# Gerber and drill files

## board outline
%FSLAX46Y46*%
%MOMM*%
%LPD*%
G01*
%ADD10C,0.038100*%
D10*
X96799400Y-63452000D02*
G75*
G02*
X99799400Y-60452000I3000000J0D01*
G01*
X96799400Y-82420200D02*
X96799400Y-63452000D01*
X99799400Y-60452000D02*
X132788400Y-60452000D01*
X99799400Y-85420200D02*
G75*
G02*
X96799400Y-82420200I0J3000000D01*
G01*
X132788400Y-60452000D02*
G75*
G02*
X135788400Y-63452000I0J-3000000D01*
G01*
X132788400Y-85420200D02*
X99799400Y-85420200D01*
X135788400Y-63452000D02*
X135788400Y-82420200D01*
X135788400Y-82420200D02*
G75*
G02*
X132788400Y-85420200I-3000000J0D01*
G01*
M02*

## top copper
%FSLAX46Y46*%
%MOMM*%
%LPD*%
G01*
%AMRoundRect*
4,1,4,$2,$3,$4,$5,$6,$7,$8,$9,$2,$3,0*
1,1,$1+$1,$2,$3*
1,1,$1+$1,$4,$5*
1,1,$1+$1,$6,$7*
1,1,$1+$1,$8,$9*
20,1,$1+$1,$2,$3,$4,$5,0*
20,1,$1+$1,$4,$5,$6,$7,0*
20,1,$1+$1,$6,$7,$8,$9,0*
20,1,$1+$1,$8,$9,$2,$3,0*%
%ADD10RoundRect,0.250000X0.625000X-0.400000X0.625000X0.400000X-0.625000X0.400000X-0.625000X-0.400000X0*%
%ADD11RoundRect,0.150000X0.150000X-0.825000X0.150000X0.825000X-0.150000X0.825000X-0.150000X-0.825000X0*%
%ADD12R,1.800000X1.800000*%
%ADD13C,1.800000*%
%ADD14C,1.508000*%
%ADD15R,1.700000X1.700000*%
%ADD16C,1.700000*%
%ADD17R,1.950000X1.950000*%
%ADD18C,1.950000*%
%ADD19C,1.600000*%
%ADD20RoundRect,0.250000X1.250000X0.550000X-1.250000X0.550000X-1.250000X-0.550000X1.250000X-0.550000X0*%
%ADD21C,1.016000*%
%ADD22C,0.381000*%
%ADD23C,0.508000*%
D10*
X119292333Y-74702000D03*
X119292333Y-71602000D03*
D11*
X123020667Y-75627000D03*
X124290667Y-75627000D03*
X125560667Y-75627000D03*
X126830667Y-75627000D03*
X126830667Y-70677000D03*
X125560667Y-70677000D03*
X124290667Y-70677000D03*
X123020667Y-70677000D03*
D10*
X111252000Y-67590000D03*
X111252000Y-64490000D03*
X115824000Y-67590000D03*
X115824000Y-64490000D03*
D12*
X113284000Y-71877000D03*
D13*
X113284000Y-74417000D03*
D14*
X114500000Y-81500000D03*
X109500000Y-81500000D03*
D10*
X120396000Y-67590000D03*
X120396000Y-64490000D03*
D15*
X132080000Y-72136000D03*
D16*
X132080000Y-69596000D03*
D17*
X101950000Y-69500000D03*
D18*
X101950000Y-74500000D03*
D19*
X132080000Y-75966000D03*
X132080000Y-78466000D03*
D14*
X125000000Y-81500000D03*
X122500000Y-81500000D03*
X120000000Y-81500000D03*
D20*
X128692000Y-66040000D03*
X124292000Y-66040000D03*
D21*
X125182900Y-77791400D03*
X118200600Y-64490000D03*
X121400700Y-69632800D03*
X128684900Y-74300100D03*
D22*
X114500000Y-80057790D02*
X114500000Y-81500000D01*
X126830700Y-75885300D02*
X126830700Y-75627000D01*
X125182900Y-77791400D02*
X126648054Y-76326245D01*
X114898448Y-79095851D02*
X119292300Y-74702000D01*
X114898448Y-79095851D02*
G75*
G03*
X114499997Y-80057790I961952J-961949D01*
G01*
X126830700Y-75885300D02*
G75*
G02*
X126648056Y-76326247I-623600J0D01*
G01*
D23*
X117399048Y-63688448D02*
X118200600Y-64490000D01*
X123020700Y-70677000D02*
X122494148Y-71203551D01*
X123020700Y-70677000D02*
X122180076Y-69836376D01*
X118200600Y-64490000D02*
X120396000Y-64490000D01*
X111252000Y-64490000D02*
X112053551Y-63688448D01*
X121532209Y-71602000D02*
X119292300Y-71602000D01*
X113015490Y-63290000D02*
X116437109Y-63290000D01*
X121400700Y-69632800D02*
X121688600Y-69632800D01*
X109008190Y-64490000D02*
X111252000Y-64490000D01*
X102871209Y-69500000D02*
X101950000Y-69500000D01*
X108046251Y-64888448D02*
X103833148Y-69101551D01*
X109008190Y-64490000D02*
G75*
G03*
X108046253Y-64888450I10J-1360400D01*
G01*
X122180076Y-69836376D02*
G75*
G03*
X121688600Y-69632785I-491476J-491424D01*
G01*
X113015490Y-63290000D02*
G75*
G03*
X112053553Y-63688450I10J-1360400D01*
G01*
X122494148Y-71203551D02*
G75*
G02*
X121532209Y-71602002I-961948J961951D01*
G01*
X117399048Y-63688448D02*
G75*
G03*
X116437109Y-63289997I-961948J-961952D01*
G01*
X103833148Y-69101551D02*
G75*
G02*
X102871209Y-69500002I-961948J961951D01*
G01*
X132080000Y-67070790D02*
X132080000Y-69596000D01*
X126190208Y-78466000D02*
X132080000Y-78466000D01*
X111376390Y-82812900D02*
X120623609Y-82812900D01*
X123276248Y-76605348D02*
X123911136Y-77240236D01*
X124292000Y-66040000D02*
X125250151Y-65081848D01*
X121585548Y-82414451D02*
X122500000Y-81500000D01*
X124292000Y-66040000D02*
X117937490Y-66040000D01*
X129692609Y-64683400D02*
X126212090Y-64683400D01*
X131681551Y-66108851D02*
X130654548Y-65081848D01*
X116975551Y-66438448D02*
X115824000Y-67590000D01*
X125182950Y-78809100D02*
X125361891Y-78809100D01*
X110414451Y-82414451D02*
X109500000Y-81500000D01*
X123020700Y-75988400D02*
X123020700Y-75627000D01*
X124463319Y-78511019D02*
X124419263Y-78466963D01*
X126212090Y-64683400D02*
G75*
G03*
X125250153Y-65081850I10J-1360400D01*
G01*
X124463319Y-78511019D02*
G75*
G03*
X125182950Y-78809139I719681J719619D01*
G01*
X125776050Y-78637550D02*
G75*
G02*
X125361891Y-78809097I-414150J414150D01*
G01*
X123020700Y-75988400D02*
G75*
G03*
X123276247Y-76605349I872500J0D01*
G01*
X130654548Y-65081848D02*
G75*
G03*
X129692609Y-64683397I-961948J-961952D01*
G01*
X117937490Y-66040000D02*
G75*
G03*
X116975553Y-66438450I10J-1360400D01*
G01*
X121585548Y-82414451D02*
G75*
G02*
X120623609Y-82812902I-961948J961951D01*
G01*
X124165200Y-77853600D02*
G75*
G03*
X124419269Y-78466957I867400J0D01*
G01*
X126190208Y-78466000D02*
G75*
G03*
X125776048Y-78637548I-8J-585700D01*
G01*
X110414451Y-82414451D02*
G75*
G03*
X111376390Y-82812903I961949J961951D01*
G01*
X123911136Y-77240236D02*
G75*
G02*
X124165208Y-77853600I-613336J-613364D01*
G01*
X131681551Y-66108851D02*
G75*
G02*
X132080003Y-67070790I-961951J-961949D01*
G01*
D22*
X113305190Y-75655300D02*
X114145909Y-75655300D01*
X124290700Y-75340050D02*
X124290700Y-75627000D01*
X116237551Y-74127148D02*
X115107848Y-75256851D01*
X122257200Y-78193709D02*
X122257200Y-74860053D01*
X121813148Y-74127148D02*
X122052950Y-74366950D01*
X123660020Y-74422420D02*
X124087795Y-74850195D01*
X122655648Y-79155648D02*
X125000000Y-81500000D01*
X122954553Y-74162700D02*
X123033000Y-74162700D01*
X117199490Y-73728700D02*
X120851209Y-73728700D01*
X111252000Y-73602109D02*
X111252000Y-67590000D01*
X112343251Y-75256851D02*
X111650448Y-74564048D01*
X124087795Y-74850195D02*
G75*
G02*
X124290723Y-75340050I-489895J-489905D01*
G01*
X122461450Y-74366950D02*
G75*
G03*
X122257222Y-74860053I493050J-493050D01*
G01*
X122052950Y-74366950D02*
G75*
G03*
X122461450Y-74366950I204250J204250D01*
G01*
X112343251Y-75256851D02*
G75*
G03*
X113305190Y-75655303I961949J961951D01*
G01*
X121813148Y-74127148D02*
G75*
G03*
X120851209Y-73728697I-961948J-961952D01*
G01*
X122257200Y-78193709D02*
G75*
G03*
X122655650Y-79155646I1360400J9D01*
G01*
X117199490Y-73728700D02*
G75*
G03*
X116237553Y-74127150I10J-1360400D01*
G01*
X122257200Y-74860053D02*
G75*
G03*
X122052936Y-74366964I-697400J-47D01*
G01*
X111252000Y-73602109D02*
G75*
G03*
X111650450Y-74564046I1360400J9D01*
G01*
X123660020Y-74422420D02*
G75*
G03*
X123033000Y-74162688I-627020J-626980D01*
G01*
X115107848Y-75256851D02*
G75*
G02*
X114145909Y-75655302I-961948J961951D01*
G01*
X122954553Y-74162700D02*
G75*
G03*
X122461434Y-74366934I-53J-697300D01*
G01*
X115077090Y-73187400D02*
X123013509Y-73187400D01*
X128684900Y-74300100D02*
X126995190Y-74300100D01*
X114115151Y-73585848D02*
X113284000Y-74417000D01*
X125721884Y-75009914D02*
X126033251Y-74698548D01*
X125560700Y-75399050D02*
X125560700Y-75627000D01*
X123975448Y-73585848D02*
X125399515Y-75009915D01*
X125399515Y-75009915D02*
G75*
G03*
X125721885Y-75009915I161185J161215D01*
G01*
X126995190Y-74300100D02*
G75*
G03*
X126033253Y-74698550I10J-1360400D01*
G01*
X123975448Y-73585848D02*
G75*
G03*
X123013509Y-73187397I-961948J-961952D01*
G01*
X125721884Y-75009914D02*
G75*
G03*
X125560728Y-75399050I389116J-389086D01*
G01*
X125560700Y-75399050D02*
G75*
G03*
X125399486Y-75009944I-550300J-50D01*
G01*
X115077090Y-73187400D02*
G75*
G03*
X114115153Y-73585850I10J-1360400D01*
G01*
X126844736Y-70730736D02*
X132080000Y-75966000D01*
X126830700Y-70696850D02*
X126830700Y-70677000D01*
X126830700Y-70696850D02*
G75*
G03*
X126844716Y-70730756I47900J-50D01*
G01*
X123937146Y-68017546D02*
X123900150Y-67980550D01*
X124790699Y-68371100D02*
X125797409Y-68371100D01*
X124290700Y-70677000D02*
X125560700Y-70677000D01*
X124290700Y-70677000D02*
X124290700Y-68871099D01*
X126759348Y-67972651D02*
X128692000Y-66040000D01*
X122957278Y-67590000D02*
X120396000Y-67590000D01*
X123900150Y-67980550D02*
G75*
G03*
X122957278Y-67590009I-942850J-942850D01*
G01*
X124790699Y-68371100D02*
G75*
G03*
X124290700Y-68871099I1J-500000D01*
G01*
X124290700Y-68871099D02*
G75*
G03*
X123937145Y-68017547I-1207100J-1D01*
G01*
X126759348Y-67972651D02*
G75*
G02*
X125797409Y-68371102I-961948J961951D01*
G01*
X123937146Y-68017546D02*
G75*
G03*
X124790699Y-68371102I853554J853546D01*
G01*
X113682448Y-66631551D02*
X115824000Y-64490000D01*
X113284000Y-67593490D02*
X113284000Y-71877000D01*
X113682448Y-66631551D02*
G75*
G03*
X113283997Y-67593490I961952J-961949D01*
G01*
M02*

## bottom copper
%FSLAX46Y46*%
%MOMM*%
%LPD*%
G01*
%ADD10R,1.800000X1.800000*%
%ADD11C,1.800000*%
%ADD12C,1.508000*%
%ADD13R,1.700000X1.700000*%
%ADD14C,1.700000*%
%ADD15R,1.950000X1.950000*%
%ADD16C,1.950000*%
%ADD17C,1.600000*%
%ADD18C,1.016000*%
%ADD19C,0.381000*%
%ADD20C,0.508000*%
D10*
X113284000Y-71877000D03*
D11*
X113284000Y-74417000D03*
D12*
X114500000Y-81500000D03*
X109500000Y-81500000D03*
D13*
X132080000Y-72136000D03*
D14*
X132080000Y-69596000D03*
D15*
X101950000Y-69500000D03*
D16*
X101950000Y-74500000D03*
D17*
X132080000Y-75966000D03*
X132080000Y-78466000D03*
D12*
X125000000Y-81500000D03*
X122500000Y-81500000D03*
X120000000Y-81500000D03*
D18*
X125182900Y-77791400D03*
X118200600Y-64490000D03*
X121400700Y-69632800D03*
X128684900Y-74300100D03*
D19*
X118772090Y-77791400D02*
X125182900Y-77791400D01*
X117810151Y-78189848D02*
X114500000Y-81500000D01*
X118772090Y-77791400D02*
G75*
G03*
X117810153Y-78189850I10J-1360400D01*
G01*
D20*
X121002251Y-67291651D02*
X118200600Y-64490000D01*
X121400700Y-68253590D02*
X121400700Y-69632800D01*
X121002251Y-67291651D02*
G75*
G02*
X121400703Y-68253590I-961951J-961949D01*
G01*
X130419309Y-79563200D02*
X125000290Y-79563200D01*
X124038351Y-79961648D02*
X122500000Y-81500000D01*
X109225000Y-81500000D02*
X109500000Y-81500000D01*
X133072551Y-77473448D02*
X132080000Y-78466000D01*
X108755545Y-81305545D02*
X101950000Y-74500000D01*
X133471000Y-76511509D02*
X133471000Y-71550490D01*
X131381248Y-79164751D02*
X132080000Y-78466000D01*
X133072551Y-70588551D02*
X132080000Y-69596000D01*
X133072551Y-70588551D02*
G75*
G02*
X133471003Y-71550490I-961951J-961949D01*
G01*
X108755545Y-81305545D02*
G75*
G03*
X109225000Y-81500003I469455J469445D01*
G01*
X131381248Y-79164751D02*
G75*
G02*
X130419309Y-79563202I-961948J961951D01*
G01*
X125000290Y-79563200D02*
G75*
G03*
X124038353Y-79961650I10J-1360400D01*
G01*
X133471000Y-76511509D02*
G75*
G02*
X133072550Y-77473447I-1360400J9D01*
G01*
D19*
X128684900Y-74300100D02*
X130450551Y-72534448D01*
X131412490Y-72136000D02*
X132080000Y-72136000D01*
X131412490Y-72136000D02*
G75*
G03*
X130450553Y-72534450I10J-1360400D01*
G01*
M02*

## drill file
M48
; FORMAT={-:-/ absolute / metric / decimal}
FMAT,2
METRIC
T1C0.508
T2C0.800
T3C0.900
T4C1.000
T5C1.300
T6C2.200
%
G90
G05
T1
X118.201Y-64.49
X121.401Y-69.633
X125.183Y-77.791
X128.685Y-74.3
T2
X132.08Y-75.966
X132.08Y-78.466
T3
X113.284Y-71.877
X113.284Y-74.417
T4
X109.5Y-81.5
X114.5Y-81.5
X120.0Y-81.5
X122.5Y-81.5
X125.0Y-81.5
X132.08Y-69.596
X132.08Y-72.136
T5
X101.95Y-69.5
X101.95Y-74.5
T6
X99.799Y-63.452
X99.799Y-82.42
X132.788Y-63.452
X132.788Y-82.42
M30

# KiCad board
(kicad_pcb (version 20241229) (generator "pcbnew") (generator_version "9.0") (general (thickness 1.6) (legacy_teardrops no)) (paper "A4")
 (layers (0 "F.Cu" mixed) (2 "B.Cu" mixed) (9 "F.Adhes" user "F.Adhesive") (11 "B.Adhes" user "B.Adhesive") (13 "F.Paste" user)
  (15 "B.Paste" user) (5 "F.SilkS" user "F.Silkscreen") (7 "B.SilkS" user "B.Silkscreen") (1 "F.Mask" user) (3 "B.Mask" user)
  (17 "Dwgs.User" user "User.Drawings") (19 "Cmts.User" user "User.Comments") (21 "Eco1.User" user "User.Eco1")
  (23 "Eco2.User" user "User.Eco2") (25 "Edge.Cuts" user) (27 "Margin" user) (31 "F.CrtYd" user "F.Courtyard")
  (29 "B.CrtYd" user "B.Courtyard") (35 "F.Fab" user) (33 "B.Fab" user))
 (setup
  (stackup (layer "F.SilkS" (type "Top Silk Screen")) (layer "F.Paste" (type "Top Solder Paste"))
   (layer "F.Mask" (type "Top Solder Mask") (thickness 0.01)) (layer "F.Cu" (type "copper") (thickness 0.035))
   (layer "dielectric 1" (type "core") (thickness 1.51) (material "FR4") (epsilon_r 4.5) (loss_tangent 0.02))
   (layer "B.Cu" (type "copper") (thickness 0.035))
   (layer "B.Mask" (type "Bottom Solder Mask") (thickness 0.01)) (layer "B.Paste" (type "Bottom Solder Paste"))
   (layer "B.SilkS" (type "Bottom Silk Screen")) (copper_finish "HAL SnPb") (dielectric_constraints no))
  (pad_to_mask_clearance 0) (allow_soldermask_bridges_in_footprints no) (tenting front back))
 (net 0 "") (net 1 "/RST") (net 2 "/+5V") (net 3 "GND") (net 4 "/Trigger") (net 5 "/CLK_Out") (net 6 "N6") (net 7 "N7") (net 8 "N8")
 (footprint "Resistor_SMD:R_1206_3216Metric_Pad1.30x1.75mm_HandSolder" (layer "F.Cu") (at 119.292333 73.152 90)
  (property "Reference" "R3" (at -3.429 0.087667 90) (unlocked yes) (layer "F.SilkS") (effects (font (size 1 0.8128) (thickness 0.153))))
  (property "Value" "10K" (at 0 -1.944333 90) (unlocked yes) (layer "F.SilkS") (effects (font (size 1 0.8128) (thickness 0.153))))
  (pad "1" smd roundrect (at -1.55 0 90) (size 1.3 1.75) (layers "F.Cu" "F.Mask" "F.Paste") (roundrect_rratio 0.192308) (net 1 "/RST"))
  (pad "2" smd roundrect (at 1.55 0 90) (size 1.3 1.75) (layers "F.Cu" "F.Mask" "F.Paste") (roundrect_rratio 0.192308) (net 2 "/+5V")))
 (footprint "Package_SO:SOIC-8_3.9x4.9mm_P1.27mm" (layer "F.Cu") (at 124.925667 73.152 90)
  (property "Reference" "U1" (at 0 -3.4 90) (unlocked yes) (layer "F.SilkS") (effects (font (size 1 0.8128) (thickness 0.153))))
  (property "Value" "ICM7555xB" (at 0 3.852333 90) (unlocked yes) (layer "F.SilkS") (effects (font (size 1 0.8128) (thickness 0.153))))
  (pad "1" smd roundrect (at -2.475 -1.905 90) (size 1.95 0.6) (layers "F.Cu" "F.Mask" "F.Paste") (roundrect_rratio 0.25) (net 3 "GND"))
  (pad "2" smd roundrect (at -2.475 -0.635 90) (size 1.95 0.6) (layers "F.Cu" "F.Mask" "F.Paste") (roundrect_rratio 0.25) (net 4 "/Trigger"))
  (pad "3" smd roundrect (at -2.475 0.635 90) (size 1.95 0.6) (layers "F.Cu" "F.Mask" "F.Paste") (roundrect_rratio 0.25) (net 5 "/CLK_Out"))
  (pad "4" smd roundrect (at -2.475 1.905 90) (size 1.95 0.6) (layers "F.Cu" "F.Mask" "F.Paste") (roundrect_rratio 0.25) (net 1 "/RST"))
  (pad "5" smd roundrect (at 2.475 1.905 90) (size 1.95 0.6) (layers "F.Cu" "F.Mask" "F.Paste") (roundrect_rratio 0.25) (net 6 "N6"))
  (pad "6" smd roundrect (at 2.475 0.635 90) (size 1.95 0.6) (layers "F.Cu" "F.Mask" "F.Paste") (roundrect_rratio 0.25) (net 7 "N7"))
  (pad "7" smd roundrect (at 2.475 -0.635 90) (size 1.95 0.6) (layers "F.Cu" "F.Mask" "F.Paste") (roundrect_rratio 0.25) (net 7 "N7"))
  (pad "8" smd roundrect (at 2.475 -1.905 90) (size 1.95 0.6) (layers "F.Cu" "F.Mask" "F.Paste") (roundrect_rratio 0.25) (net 2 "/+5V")))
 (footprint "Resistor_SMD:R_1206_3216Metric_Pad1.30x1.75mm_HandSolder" (layer "F.Cu") (at 111.252 66.04 90)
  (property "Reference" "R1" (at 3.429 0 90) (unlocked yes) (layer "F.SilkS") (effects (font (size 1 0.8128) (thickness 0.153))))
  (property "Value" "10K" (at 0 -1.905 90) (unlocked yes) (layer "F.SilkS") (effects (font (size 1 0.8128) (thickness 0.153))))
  (pad "1" smd roundrect (at -1.55 0 90) (size 1.3 1.75) (layers "F.Cu" "F.Mask" "F.Paste") (roundrect_rratio 0.192308) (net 4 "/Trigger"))
  (pad "2" smd roundrect (at 1.55 0 90) (size 1.3 1.75) (layers "F.Cu" "F.Mask" "F.Paste") (roundrect_rratio 0.192308) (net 2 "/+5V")))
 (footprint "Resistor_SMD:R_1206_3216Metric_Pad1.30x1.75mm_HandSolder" (layer "F.Cu") (at 115.824 66.04 90)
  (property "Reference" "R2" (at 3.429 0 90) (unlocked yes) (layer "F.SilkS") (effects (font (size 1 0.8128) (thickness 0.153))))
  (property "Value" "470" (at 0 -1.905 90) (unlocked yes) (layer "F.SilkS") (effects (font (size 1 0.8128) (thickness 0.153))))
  (pad "1" smd roundrect (at -1.55 0 90) (size 1.3 1.75) (layers "F.Cu" "F.Mask" "F.Paste") (roundrect_rratio 0.192308) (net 3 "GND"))
  (pad "2" smd roundrect (at 1.55 0 90) (size 1.3 1.75) (layers "F.Cu" "F.Mask" "F.Paste") (roundrect_rratio 0.192308) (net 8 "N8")))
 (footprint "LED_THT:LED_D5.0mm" (layer "F.Cu") (at 113.284 71.877 -90)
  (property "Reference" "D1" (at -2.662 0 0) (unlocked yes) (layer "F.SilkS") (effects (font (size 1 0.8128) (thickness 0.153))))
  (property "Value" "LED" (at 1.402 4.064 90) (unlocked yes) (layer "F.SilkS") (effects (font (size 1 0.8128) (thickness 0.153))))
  (pad "1" thru_hole rect (at 0 0 270) (size 1.8 1.8) (drill 0.9) (layers "*.Cu" "*.Mask") (remove_unused_layers no) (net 8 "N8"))
  (pad "2" thru_hole circle (at 2.54 0 270) (size 1.8 1.8) (drill 0.9) (layers "*.Cu" "*.Mask") (remove_unused_layers no) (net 5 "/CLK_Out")))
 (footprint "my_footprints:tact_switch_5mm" (layer "F.Cu") (at 112 81.5 180)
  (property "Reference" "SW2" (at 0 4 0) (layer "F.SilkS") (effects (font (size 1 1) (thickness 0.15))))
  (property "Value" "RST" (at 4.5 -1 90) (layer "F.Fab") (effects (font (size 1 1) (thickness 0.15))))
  (pad "1" thru_hole circle (at -2.5 0 180) (size 1.508 1.508) (drill 1) (layers "*.Cu" "*.Mask") (remove_unused_layers no) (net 1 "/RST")
   (solder_mask_margin 0.102))
  (pad "2" thru_hole circle (at 2.5 0 180) (size 1.508 1.508) (drill 1) (layers "*.Cu" "*.Mask") (remove_unused_layers no) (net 3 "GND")
   (solder_mask_margin 0.102)))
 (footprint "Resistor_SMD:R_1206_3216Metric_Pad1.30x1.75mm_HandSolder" (layer "F.Cu") (at 120.396 66.04 90)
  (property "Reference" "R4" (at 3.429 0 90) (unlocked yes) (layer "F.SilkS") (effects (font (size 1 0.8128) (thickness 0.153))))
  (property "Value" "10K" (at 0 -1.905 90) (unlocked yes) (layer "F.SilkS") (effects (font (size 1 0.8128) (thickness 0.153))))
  (pad "1" smd roundrect (at -1.55 0 90) (size 1.3 1.75) (layers "F.Cu" "F.Mask" "F.Paste") (roundrect_rratio 0.192308) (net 7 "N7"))
  (pad "2" smd roundrect (at 1.55 0 90) (size 1.3 1.75) (layers "F.Cu" "F.Mask" "F.Paste") (roundrect_rratio 0.192308) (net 2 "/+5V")))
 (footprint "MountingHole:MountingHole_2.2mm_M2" (layer "F.Cu") (at 99.7994 63.452)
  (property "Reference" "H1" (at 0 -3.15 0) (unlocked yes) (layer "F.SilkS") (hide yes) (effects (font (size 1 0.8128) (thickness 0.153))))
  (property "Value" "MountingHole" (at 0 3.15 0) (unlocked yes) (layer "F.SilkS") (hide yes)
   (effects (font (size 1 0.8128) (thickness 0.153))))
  (pad "" np_thru_hole circle (at 0 0) (size 2.2 2.2) (drill 2.2) (layers "*.Cu" "*.Mask")))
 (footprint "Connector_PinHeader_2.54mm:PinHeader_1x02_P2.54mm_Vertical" (layer "F.Cu") (at 132.08 72.136 180)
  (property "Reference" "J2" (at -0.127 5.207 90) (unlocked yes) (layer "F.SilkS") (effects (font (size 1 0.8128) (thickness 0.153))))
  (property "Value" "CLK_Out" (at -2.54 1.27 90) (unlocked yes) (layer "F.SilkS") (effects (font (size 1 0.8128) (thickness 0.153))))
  (pad "1" thru_hole rect (at 0 0 180) (size 1.7 1.7) (drill 1) (layers "*.Cu" "*.Mask") (remove_unused_layers no) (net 5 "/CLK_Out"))
  (pad "2" thru_hole circle (at 0 2.54 180) (size 1.7 1.7) (drill 1) (layers "*.Cu" "*.Mask") (remove_unused_layers no) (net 3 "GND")))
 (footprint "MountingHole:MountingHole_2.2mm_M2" (layer "F.Cu") (at 132.7884 82.4202)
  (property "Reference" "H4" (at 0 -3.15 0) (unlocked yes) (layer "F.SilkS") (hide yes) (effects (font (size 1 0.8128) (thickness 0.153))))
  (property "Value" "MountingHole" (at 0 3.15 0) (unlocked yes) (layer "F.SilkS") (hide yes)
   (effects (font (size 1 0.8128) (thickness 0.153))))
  (pad "" np_thru_hole circle (at 0 0) (size 2.2 2.2) (drill 2.2) (layers "*.Cu" "*.Mask")))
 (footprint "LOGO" (layer "F.Cu") (at 105.5 63.5)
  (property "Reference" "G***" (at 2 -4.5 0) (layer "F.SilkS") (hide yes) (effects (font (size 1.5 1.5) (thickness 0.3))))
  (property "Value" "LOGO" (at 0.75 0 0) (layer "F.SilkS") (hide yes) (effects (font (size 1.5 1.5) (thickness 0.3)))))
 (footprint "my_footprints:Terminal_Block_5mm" (layer "F.Cu") (at 101.95 72 -90)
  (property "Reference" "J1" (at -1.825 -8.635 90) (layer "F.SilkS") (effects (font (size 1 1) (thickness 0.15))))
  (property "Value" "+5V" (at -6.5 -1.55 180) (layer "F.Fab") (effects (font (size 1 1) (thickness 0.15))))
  (pad "1" thru_hole rect (at -2.5 0 270) (size 1.95 1.95) (drill 1.3) (layers "*.Cu" "*.Mask") (remove_unused_layers no) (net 2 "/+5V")
   (solder_mask_margin 0.102))
  (pad "2" thru_hole circle (at 2.5 0 270) (size 1.95 1.95) (drill 1.3) (layers "*.Cu" "*.Mask") (remove_unused_layers no) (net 3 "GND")
   (solder_mask_margin 0.102)))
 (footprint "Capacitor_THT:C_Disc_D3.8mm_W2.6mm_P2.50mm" (layer "F.Cu") (at 132.08 75.966 -90)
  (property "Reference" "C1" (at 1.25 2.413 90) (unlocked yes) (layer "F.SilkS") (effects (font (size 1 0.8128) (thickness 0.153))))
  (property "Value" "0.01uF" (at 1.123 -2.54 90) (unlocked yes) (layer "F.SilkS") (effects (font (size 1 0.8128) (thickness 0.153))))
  (pad "1" thru_hole circle (at 0 0 270) (size 1.6 1.6) (drill 0.8) (layers "*.Cu" "*.Mask") (remove_unused_layers no) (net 6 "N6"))
  (pad "2" thru_hole circle (at 2.5 0 270) (size 1.6 1.6) (drill 0.8) (layers "*.Cu" "*.Mask") (remove_unused_layers no) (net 3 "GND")))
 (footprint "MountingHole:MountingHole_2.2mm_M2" (layer "F.Cu") (at 132.7884 63.452)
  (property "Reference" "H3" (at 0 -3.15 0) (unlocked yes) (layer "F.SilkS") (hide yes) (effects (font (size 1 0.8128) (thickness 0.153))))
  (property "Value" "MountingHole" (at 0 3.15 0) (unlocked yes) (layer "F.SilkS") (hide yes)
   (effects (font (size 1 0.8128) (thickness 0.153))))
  (pad "" np_thru_hole circle (at 0 0) (size 2.2 2.2) (drill 2.2) (layers "*.Cu" "*.Mask")))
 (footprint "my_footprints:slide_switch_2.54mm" (layer "F.Cu") (at 122.5 81.5 180)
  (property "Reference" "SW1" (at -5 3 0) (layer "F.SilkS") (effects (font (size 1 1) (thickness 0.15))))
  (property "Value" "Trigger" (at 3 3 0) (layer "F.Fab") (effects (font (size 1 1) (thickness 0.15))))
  (pad "1" thru_hole circle (at -2.5 0 180) (size 1.508 1.508) (drill 1) (layers "*.Cu" "*.Mask") (remove_unused_layers no)
   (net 4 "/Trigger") (solder_mask_margin 0.102))
  (pad "2" thru_hole circle (at 0 0 180) (size 1.508 1.508) (drill 1) (layers "*.Cu" "*.Mask") (remove_unused_layers no) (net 3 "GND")
   (solder_mask_margin 0.102))
  (pad "3" thru_hole circle (at 2.5 0 180) (size 1.508 1.508) (drill 1) (layers "*.Cu" "*.Mask") (remove_unused_layers no)
   (solder_mask_margin 0.102)))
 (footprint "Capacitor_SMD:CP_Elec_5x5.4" (layer "F.Cu") (at 126.492 66.04 180)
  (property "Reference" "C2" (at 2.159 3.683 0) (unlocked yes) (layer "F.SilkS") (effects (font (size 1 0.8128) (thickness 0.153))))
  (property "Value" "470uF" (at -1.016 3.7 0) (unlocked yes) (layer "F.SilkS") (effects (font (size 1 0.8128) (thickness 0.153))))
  (pad "1" smd roundrect (at -2.2 0 180) (size 3 1.6) (layers "F.Cu" "F.Mask" "F.Paste") (roundrect_rratio 0.15625) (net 7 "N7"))
  (pad "2" smd roundrect (at 2.2 0 180) (size 3 1.6) (layers "F.Cu" "F.Mask" "F.Paste") (roundrect_rratio 0.15625) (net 3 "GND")))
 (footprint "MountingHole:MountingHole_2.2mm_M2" (layer "F.Cu") (at 99.7994 82.4202)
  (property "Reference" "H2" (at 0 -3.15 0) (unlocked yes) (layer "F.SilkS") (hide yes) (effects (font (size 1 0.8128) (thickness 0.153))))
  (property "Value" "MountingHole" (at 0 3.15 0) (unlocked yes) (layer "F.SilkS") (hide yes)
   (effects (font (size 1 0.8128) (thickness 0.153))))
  (pad "" np_thru_hole circle (at 0 0) (size 2.2 2.2) (drill 2.2) (layers "*.Cu" "*.Mask")))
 (gr_arc (start 96.7994 63.452) (mid 97.67808 61.33068) (end 99.7994 60.452) (stroke (width 0.0381) (type default)) (layer "Edge.Cuts"))
 (gr_line (start 96.7994 82.4202) (end 96.7994 63.452) (stroke (width 0.0381) (type default)) (layer "Edge.Cuts"))
 (gr_line (start 99.7994 60.452) (end 132.7884 60.452) (stroke (width 0.0381) (type default)) (layer "Edge.Cuts"))
 (gr_arc (start 99.7994 85.4202) (mid 97.67808 84.54152) (end 96.7994 82.4202) (stroke (width 0.0381) (type default)) (layer "Edge.Cuts"))
 (gr_arc (start 132.7884 60.452) (mid 134.90972 61.33068) (end 135.7884 63.452) (stroke (width 0.0381) (type default)) (layer "Edge.Cuts"))
 (gr_line (start 132.7884 85.4202) (end 99.7994 85.4202) (stroke (width 0.0381) (type default)) (layer "Edge.Cuts"))
 (gr_line (start 135.7884 63.452) (end 135.7884 82.4202) (stroke (width 0.0381) (type default)) (layer "Edge.Cuts"))
 (gr_arc (start 135.7884 82.4202) (mid 134.90972 84.54152) (end 132.7884 85.4202) (stroke (width 0.0381) (type default)) (layer "Edge.Cuts"))
 (segment (start 114.500000 80.057790) (end 114.500000 81.500000) (width 0.381000) (layer "F.Cu") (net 1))
 (segment (start 126.830700 75.885300) (end 126.830700 75.627000) (width 0.381000) (layer "F.Cu") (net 1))
 (segment (start 125.182900 77.791400) (end 126.648054 76.326245) (width 0.381000) (layer "F.Cu") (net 1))
 (segment (start 114.898448 79.095851) (end 119.292300 74.702000) (width 0.381000) (layer "F.Cu") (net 1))
 (arc (start 114.898448 79.095851) (mid 114.603553 79.537192) (end 114.500000 80.057790) (width 0.381000) (layer "F.Cu") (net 1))
 (arc (start 126.830700 75.885300) (mid 126.783231 76.123937) (end 126.648054 76.326245) (width 0.381000) (layer "F.Cu") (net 1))
 (segment (start 118.772090 77.791400) (end 125.182900 77.791400) (width 0.381000) (layer "B.Cu") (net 1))
 (segment (start 117.810151 78.189848) (end 114.500000 81.500000) (width 0.381000) (layer "B.Cu") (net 1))
 (arc (start 118.772090 77.791400) (mid 118.251492 77.894953) (end 117.810151 78.189848) (width 0.381000) (layer "B.Cu") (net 1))
 (segment (start 117.399048 63.688448) (end 118.200600 64.490000) (width 0.508000) (layer "F.Cu") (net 2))
 (segment (start 123.020700 70.677000) (end 122.494148 71.203551) (width 0.508000) (layer "F.Cu") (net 2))
 (segment (start 123.020700 70.677000) (end 122.180076 69.836376) (width 0.508000) (layer "F.Cu") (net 2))
 (segment (start 118.200600 64.490000) (end 120.396000 64.490000) (width 0.508000) (layer "F.Cu") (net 2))
 (segment (start 111.252000 64.490000) (end 112.053551 63.688448) (width 0.508000) (layer "F.Cu") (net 2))
 (segment (start 121.532209 71.602000) (end 119.292300 71.602000) (width 0.508000) (layer "F.Cu") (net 2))
 (segment (start 113.015490 63.290000) (end 116.437109 63.290000) (width 0.508000) (layer "F.Cu") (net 2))
 (segment (start 121.400700 69.632800) (end 121.688600 69.632800) (width 0.508000) (layer "F.Cu") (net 2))
 (segment (start 109.008190 64.490000) (end 111.252000 64.490000) (width 0.508000) (layer "F.Cu") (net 2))
 (segment (start 102.871209 69.500000) (end 101.950000 69.500000) (width 0.508000) (layer "F.Cu") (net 2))
 (segment (start 108.046251 64.888448) (end 103.833148 69.101551) (width 0.508000) (layer "F.Cu") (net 2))
 (arc (start 109.008190 64.490000) (mid 108.487592 64.593553) (end 108.046251 64.888448) (width 0.508000) (layer "F.Cu") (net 2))
 (arc (start 122.180076 69.836376) (mid 121.954584 69.685707) (end 121.688600 69.632800) (width 0.508000) (layer "F.Cu") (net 2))
 (arc (start 113.015490 63.290000) (mid 112.494892 63.393553) (end 112.053551 63.688448) (width 0.508000) (layer "F.Cu") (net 2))
 (arc (start 122.494148 71.203551) (mid 122.052806 71.498446) (end 121.532209 71.602000) (width 0.508000) (layer "F.Cu") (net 2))
 (arc (start 117.399048 63.688448) (mid 116.957706 63.393553) (end 116.437109 63.290000) (width 0.508000) (layer "F.Cu") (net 2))
 (arc (start 103.833148 69.101551) (mid 103.391806 69.396446) (end 102.871209 69.500000) (width 0.508000) (layer "F.Cu") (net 2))
 (segment (start 121.002251 67.291651) (end 118.200600 64.490000) (width 0.508000) (layer "B.Cu") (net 2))
 (segment (start 121.400700 68.253590) (end 121.400700 69.632800) (width 0.508000) (layer "B.Cu") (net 2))
 (arc (start 121.002251 67.291651) (mid 121.297146 67.732992) (end 121.400700 68.253590) (width 0.508000) (layer "B.Cu") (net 2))
 (segment (start 132.080000 67.070790) (end 132.080000 69.596000) (width 0.508000) (layer "F.Cu") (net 3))
 (segment (start 126.190208 78.466000) (end 132.080000 78.466000) (width 0.508000) (layer "F.Cu") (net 3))
 (segment (start 111.376390 82.812900) (end 120.623609 82.812900) (width 0.508000) (layer "F.Cu") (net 3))
 (segment (start 123.276248 76.605348) (end 123.911136 77.240236) (width 0.508000) (layer "F.Cu") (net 3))
 (segment (start 124.292000 66.040000) (end 125.250151 65.081848) (width 0.508000) (layer "F.Cu") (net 3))
 (segment (start 121.585548 82.414451) (end 122.500000 81.500000) (width 0.508000) (layer "F.Cu") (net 3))
 (segment (start 124.292000 66.040000) (end 117.937490 66.040000) (width 0.508000) (layer "F.Cu") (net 3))
 (segment (start 129.692609 64.683400) (end 126.212090 64.683400) (width 0.508000) (layer "F.Cu") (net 3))
 (segment (start 131.681551 66.108851) (end 130.654548 65.081848) (width 0.508000) (layer "F.Cu") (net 3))
 (segment (start 116.975551 66.438448) (end 115.824000 67.590000) (width 0.508000) (layer "F.Cu") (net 3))
 (segment (start 125.182950 78.809100) (end 125.361891 78.809100) (width 0.508000) (layer "F.Cu") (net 3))
 (segment (start 110.414451 82.414451) (end 109.500000 81.500000) (width 0.508000) (layer "F.Cu") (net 3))
 (segment (start 123.020700 75.988400) (end 123.020700 75.627000) (width 0.508000) (layer "F.Cu") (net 3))
 (segment (start 124.463319 78.511019) (end 124.419263 78.466963) (width 0.508000) (layer "F.Cu") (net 3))
 (arc (start 126.212090 64.683400) (mid 125.691492 64.786953) (end 125.250151 65.081848) (width 0.508000) (layer "F.Cu") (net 3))
 (arc (start 124.463319 78.511019) (mid 124.793488 78.731631) (end 125.182950 78.809100) (width 0.508000) (layer "F.Cu") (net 3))
 (arc (start 125.776050 78.637550) (mid 125.586032 78.764515) (end 125.361891 78.809100) (width 0.508000) (layer "F.Cu") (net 3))
 (arc (start 123.020700 75.988400) (mid 123.087114 76.322289) (end 123.276248 76.605348) (width 0.508000) (layer "F.Cu") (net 3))
 (arc (start 130.654548 65.081848) (mid 130.213206 64.786953) (end 129.692609 64.683400) (width 0.508000) (layer "F.Cu") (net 3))
 (arc (start 117.937490 66.040000) (mid 117.416892 66.143553) (end 116.975551 66.438448) (width 0.508000) (layer "F.Cu") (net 3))
 (arc (start 121.585548 82.414451) (mid 121.144206 82.709346) (end 120.623609 82.812900) (width 0.508000) (layer "F.Cu") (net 3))
 (arc (start 124.165200 77.853600) (mid 124.231228 78.185549) (end 124.419263 78.466963) (width 0.508000) (layer "F.Cu") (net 3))
 (arc (start 126.190208 78.466000) (mid 125.966067 78.510584) (end 125.776050 78.637550) (width 0.508000) (layer "F.Cu") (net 3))
 (arc (start 110.414451 82.414451) (mid 110.855792 82.709346) (end 111.376390 82.812900) (width 0.508000) (layer "F.Cu") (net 3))
 (arc (start 123.911136 77.240236) (mid 124.099170 77.521649) (end 124.165200 77.853600) (width 0.508000) (layer "F.Cu") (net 3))
 (arc (start 131.681551 66.108851) (mid 131.976446 66.550192) (end 132.080000 67.070790) (width 0.508000) (layer "F.Cu") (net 3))
 (segment (start 130.419309 79.563200) (end 125.000290 79.563200) (width 0.508000) (layer "B.Cu") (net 3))
 (segment (start 124.038351 79.961648) (end 122.500000 81.500000) (width 0.508000) (layer "B.Cu") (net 3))
 (segment (start 109.225000 81.500000) (end 109.500000 81.500000) (width 0.508000) (layer "B.Cu") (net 3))
 (segment (start 133.072551 77.473448) (end 132.080000 78.466000) (width 0.508000) (layer "B.Cu") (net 3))
 (segment (start 108.755545 81.305545) (end 101.950000 74.500000) (width 0.508000) (layer "B.Cu") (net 3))
 (segment (start 133.471000 76.511509) (end 133.471000 71.550490) (width 0.508000) (layer "B.Cu") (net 3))
 (segment (start 131.381248 79.164751) (end 132.080000 78.466000) (width 0.508000) (layer "B.Cu") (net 3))
 (segment (start 133.072551 70.588551) (end 132.080000 69.596000) (width 0.508000) (layer "B.Cu") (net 3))
 (arc (start 133.072551 70.588551) (mid 133.367446 71.029892) (end 133.471000 71.550490) (width 0.508000) (layer "B.Cu") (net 3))
 (arc (start 108.755545 81.305545) (mid 108.970932 81.449462) (end 109.225000 81.500000) (width 0.508000) (layer "B.Cu") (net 3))
 (arc (start 131.381248 79.164751) (mid 130.939906 79.459646) (end 130.419309 79.563200) (width 0.508000) (layer "B.Cu") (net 3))
 (arc (start 125.000290 79.563200) (mid 124.479692 79.666753) (end 124.038351 79.961648) (width 0.508000) (layer "B.Cu") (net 3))
 (arc (start 133.471000 76.511509) (mid 133.367446 77.032106) (end 133.072551 77.473448) (width 0.508000) (layer "B.Cu") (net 3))
 (segment (start 113.305190 75.655300) (end 114.145909 75.655300) (width 0.381000) (layer "F.Cu") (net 4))
 (segment (start 124.290700 75.340050) (end 124.290700 75.627000) (width 0.381000) (layer "F.Cu") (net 4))
 (segment (start 116.237551 74.127148) (end 115.107848 75.256851) (width 0.381000) (layer "F.Cu") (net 4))
 (segment (start 122.257200 78.193709) (end 122.257200 74.860053) (width 0.381000) (layer "F.Cu") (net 4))
 (segment (start 121.813148 74.127148) (end 122.052950 74.366950) (width 0.381000) (layer "F.Cu") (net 4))
 (segment (start 123.660020 74.422420) (end 124.087795 74.850195) (width 0.381000) (layer "F.Cu") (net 4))
 (segment (start 122.655648 79.155648) (end 125.000000 81.500000) (width 0.381000) (layer "F.Cu") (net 4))
 (segment (start 122.954553 74.162700) (end 123.033000 74.162700) (width 0.381000) (layer "F.Cu") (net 4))
 (segment (start 117.199490 73.728700) (end 120.851209 73.728700) (width 0.381000) (layer "F.Cu") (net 4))
 (segment (start 111.252000 73.602109) (end 111.252000 67.590000) (width 0.381000) (layer "F.Cu") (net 4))
 (segment (start 112.343251 75.256851) (end 111.650448 74.564048) (width 0.381000) (layer "F.Cu") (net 4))
 (arc (start 124.087795 74.850195) (mid 124.237966 75.074942) (end 124.290700 75.340050) (width 0.381000) (layer "F.Cu") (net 4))
 (arc (start 122.461450 74.366950) (mid 122.310282 74.593187) (end 122.257200 74.860053) (width 0.381000) (layer "F.Cu") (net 4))
 (arc (start 122.052950 74.366950) (mid 122.257200 74.451553) (end 122.461450 74.366950) (width 0.381000) (layer "F.Cu") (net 4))
 (arc (start 112.343251 75.256851) (mid 112.784592 75.551746) (end 113.305190 75.655300) (width 0.381000) (layer "F.Cu") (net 4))
 (arc (start 121.813148 74.127148) (mid 121.371806 73.832253) (end 120.851209 73.728700) (width 0.381000) (layer "F.Cu") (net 4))
 (arc (start 122.257200 78.193709) (mid 122.360753 78.714306) (end 122.655648 79.155648) (width 0.381000) (layer "F.Cu") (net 4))
 (arc (start 117.199490 73.728700) (mid 116.678892 73.832253) (end 116.237551 74.127148) (width 0.381000) (layer "F.Cu") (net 4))
 (arc (start 122.257200 74.860053) (mid 122.204117 74.593187) (end 122.052950 74.366950) (width 0.381000) (layer "F.Cu") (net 4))
 (arc (start 111.252000 73.602109) (mid 111.355553 74.122706) (end 111.650448 74.564048) (width 0.381000) (layer "F.Cu") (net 4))
 (arc (start 123.660020 74.422420) (mid 123.372340 74.230199) (end 123.033000 74.162700) (width 0.381000) (layer "F.Cu") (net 4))
 (arc (start 115.107848 75.256851) (mid 114.666506 75.551746) (end 114.145909 75.655300) (width 0.381000) (layer "F.Cu") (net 4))
 (arc (start 122.954553 74.162700) (mid 122.687687 74.215782) (end 122.461450 74.366950) (width 0.381000) (layer "F.Cu") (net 4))
 (segment (start 115.077090 73.187400) (end 123.013509 73.187400) (width 0.381000) (layer "F.Cu") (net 5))
 (segment (start 128.684900 74.300100) (end 126.995190 74.300100) (width 0.381000) (layer "F.Cu") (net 5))
 (segment (start 114.115151 73.585848) (end 113.284000 74.417000) (width 0.381000) (layer "F.Cu") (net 5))
 (segment (start 125.721884 75.009914) (end 126.033251 74.698548) (width 0.381000) (layer "F.Cu") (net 5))
 (segment (start 125.560700 75.399050) (end 125.560700 75.627000) (width 0.381000) (layer "F.Cu") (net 5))
 (segment (start 123.975448 73.585848) (end 125.399515 75.009915) (width 0.381000) (layer "F.Cu") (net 5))
 (arc (start 125.399515 75.009915) (mid 125.560699 75.076679) (end 125.721884 75.009914) (width 0.381000) (layer "F.Cu") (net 5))
 (arc (start 126.995190 74.300100) (mid 126.474592 74.403653) (end 126.033251 74.698548) (width 0.381000) (layer "F.Cu") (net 5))
 (arc (start 123.975448 73.585848) (mid 123.534106 73.290953) (end 123.013509 73.187400) (width 0.381000) (layer "F.Cu") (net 5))
 (arc (start 125.721884 75.009914) (mid 125.602590 75.188451) (end 125.560700 75.399050) (width 0.381000) (layer "F.Cu") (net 5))
 (arc (start 125.560700 75.399050) (mid 125.518809 75.188451) (end 125.399515 75.009915) (width 0.381000) (layer "F.Cu") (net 5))
 (arc (start 115.077090 73.187400) (mid 114.556492 73.290953) (end 114.115151 73.585848) (width 0.381000) (layer "F.Cu") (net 5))
 (segment (start 128.684900 74.300100) (end 130.450551 72.534448) (width 0.381000) (layer "B.Cu") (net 5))
 (segment (start 131.412490 72.136000) (end 132.080000 72.136000) (width 0.381000) (layer "B.Cu") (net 5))
 (arc (start 131.412490 72.136000) (mid 130.891892 72.239553) (end 130.450551 72.534448) (width 0.381000) (layer "B.Cu") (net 5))
 (segment (start 126.844736 70.730736) (end 132.080000 75.966000) (width 0.381000) (layer "F.Cu") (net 6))
 (segment (start 126.830700 70.696850) (end 126.830700 70.677000) (width 0.381000) (layer "F.Cu") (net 6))
 (arc (start 126.830700 70.696850) (mid 126.834347 70.715188) (end 126.844736 70.730736) (width 0.381000) (layer "F.Cu") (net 6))
 (segment (start 123.937146 68.017546) (end 123.900150 67.980550) (width 0.381000) (layer "F.Cu") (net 7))
 (segment (start 124.790699 68.371100) (end 125.797409 68.371100) (width 0.381000) (layer "F.Cu") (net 7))
 (segment (start 124.290700 70.677000) (end 125.560700 70.677000) (width 0.381000) (layer "F.Cu") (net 7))
 (segment (start 124.290700 70.677000) (end 124.290700 68.871099) (width 0.381000) (layer "F.Cu") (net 7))
 (segment (start 126.759348 67.972651) (end 128.692000 66.040000) (width 0.381000) (layer "F.Cu") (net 7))
 (segment (start 122.957278 67.590000) (end 120.396000 67.590000) (width 0.381000) (layer "F.Cu") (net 7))
 (arc (start 123.900150 67.980550) (mid 123.467556 67.691500) (end 122.957278 67.590000) (width 0.381000) (layer "F.Cu") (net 7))
 (arc (start 124.790699 68.371100) (mid 124.437146 68.517546) (end 124.290700 68.871099) (width 0.381000) (layer "F.Cu") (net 7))
 (arc (start 124.290700 68.871099) (mid 124.198814 68.409159) (end 123.937146 68.017546) (width 0.381000) (layer "F.Cu") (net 7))
 (arc (start 126.759348 67.972651) (mid 126.318006 68.267546) (end 125.797409 68.371100) (width 0.381000) (layer "F.Cu") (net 7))
 (arc (start 123.937146 68.017546) (mid 124.328759 68.279214) (end 124.790699 68.371100) (width 0.381000) (layer "F.Cu") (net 7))
 (segment (start 113.682448 66.631551) (end 115.824000 64.490000) (width 0.381000) (layer "F.Cu") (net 8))
 (segment (start 113.284000 67.593490) (end 113.284000 71.877000) (width 0.381000) (layer "F.Cu") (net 8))
 (arc (start 113.682448 66.631551) (mid 113.387553 67.072892) (end 113.284000 67.593490) (width 0.381000) (layer "F.Cu") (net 8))
 (via (at 125.182900 77.791400) (size 1.016000) (drill 0.508000) (layers "F.Cu" "B.Cu") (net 1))
 (via (at 118.200600 64.490000) (size 1.016000) (drill 0.508000) (layers "F.Cu" "B.Cu") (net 2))
 (via (at 121.400700 69.632800) (size 1.016000) (drill 0.508000) (layers "F.Cu" "B.Cu") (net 2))
 (via (at 128.684900 74.300100) (size 1.016000) (drill 0.508000) (layers "F.Cu" "B.Cu") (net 5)))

